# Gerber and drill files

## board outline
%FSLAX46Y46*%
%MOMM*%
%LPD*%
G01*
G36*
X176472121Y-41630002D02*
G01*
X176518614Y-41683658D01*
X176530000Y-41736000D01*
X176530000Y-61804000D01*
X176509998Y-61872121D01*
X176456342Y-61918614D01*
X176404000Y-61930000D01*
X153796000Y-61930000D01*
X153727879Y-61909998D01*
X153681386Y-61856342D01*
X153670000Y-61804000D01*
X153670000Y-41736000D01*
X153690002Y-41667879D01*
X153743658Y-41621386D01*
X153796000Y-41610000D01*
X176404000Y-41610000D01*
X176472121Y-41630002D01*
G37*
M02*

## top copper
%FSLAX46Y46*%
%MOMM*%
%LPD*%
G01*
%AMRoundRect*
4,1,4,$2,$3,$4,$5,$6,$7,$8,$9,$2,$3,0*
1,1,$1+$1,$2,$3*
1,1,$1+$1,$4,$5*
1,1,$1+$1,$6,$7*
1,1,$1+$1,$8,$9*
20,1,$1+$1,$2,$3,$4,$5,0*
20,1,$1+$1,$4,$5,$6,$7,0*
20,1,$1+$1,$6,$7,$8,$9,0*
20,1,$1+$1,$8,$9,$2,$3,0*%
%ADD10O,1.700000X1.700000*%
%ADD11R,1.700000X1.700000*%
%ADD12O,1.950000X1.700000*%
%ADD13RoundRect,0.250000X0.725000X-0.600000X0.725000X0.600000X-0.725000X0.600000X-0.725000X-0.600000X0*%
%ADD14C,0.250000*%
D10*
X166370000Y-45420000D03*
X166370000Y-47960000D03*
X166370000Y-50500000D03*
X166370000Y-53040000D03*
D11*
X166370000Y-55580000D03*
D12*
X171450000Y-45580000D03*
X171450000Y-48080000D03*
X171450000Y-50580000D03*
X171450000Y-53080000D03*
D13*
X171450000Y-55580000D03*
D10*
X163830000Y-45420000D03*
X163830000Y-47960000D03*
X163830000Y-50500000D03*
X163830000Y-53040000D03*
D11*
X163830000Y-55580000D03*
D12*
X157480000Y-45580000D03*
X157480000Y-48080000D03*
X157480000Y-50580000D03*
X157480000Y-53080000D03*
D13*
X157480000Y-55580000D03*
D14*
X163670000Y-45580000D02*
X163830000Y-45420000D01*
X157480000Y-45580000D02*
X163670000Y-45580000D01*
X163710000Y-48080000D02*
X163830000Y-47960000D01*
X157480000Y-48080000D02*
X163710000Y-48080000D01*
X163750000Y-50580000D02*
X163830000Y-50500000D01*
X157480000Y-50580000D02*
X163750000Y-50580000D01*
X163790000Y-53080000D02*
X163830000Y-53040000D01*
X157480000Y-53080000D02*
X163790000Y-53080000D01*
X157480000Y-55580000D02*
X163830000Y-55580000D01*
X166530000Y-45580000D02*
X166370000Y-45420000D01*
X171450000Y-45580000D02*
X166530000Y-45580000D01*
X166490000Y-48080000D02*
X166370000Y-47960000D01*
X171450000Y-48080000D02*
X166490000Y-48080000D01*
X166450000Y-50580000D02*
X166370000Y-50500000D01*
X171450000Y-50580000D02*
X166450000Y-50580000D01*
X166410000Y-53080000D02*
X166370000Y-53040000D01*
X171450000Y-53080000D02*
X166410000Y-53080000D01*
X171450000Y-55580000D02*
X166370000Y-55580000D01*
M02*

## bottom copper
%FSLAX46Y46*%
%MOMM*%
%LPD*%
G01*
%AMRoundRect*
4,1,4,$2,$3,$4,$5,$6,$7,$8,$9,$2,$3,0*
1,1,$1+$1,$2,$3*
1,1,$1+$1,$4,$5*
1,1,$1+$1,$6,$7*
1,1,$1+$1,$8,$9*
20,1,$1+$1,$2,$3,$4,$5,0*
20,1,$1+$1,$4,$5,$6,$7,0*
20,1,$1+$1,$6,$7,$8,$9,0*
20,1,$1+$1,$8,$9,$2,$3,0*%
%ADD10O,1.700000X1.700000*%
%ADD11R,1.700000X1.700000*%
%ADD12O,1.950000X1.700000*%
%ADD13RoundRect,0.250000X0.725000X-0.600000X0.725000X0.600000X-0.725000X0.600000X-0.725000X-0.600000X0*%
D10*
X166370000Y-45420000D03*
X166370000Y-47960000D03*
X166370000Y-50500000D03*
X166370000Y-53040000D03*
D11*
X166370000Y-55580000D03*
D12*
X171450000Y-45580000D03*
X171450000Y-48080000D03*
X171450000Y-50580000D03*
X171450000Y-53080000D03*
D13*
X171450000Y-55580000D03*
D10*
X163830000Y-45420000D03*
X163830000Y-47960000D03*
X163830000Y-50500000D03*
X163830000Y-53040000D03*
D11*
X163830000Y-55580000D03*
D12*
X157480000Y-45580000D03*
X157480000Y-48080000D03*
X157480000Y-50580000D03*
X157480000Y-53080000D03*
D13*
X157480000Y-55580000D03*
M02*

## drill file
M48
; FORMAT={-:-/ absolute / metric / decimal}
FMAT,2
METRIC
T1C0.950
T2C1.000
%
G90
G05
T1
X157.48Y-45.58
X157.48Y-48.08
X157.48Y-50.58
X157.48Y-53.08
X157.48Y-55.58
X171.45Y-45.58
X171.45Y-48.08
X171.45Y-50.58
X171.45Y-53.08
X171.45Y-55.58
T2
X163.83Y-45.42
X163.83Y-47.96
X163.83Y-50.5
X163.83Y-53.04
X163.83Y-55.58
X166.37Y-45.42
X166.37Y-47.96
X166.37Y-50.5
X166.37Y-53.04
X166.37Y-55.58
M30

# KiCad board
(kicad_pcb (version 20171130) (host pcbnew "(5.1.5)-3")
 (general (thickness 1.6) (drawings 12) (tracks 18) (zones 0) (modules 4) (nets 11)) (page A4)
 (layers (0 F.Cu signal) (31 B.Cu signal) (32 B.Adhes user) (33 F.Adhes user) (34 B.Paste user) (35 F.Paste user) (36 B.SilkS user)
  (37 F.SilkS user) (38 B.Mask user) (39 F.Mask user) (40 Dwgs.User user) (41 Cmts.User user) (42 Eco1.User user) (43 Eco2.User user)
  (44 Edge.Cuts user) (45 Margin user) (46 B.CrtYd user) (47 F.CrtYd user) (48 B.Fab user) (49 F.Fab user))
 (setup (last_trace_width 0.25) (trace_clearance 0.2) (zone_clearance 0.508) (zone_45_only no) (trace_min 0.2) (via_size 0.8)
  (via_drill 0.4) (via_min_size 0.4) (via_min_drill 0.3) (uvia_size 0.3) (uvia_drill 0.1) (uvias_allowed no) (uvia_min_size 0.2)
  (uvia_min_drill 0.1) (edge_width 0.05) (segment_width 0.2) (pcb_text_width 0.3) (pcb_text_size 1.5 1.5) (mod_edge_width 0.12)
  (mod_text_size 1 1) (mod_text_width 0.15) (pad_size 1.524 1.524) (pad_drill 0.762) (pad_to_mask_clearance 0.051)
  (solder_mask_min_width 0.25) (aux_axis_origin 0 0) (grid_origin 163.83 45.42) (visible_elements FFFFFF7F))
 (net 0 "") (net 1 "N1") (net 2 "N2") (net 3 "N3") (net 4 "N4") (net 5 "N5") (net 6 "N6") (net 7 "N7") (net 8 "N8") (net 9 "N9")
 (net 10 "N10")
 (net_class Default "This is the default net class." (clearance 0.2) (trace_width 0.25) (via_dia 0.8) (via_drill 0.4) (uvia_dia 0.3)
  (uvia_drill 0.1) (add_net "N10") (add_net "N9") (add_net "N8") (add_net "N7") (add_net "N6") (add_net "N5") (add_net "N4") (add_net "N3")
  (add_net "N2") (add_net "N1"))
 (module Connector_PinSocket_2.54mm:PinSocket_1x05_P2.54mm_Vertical (layer B.Cu) (at 166.37 55.58)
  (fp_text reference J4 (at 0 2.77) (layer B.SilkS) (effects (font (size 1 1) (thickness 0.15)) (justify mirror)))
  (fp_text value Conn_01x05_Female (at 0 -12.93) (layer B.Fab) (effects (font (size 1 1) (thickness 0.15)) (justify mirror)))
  (pad 5 thru_hole oval (at 0 -10.16) (size 1.7 1.7) (drill 1) (layers *.Cu *.Mask) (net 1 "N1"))
  (pad 4 thru_hole oval (at 0 -7.62) (size 1.7 1.7) (drill 1) (layers *.Cu *.Mask) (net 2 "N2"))
  (pad 3 thru_hole oval (at 0 -5.08) (size 1.7 1.7) (drill 1) (layers *.Cu *.Mask) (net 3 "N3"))
  (pad 2 thru_hole oval (at 0 -2.54) (size 1.7 1.7) (drill 1) (layers *.Cu *.Mask) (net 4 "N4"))
  (pad 1 thru_hole rect (at 0 0) (size 1.7 1.7) (drill 1) (layers *.Cu *.Mask) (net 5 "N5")))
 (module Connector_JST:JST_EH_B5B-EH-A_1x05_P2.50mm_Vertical (layer F.Cu) (at 171.45 55.58 90)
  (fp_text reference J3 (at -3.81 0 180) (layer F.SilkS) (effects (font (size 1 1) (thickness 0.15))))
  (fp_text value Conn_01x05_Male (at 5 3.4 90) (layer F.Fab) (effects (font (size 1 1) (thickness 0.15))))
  (pad 5 thru_hole oval (at 10 0 90) (size 1.7 1.95) (drill 0.95) (layers *.Cu *.Mask) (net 1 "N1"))
  (pad 4 thru_hole oval (at 7.5 0 90) (size 1.7 1.95) (drill 0.95) (layers *.Cu *.Mask) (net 2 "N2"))
  (pad 3 thru_hole oval (at 5 0 90) (size 1.7 1.95) (drill 0.95) (layers *.Cu *.Mask) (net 3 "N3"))
  (pad 2 thru_hole oval (at 2.5 0 90) (size 1.7 1.95) (drill 0.95) (layers *.Cu *.Mask) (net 4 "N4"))
  (pad 1 thru_hole roundrect (at 0 0 90) (size 1.7 1.95) (drill 0.95) (layers *.Cu *.Mask) (roundrect_rratio 0.147059) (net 5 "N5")))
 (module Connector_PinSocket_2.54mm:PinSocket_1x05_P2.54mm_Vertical (layer B.Cu) (at 163.83 55.58)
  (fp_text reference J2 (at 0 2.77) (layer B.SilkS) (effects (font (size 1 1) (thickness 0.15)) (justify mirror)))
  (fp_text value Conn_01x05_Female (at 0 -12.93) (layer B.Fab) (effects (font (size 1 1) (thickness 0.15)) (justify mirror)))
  (pad 5 thru_hole oval (at 0 -10.16) (size 1.7 1.7) (drill 1) (layers *.Cu *.Mask) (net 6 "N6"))
  (pad 4 thru_hole oval (at 0 -7.62) (size 1.7 1.7) (drill 1) (layers *.Cu *.Mask) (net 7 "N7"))
  (pad 3 thru_hole oval (at 0 -5.08) (size 1.7 1.7) (drill 1) (layers *.Cu *.Mask) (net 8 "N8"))
  (pad 2 thru_hole oval (at 0 -2.54) (size 1.7 1.7) (drill 1) (layers *.Cu *.Mask) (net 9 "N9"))
  (pad 1 thru_hole rect (at 0 0) (size 1.7 1.7) (drill 1) (layers *.Cu *.Mask) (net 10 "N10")))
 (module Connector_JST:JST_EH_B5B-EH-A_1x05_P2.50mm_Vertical (layer F.Cu) (at 157.48 55.58 90)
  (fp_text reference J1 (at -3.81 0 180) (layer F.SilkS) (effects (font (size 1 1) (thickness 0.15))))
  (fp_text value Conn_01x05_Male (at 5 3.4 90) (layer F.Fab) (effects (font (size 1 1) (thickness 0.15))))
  (pad 5 thru_hole oval (at 10 0 90) (size 1.7 1.95) (drill 0.95) (layers *.Cu *.Mask) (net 6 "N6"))
  (pad 4 thru_hole oval (at 7.5 0 90) (size 1.7 1.95) (drill 0.95) (layers *.Cu *.Mask) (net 7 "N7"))
  (pad 3 thru_hole oval (at 5 0 90) (size 1.7 1.95) (drill 0.95) (layers *.Cu *.Mask) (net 8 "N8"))
  (pad 2 thru_hole oval (at 2.5 0 90) (size 1.7 1.95) (drill 0.95) (layers *.Cu *.Mask) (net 9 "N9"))
  (pad 1 thru_hole roundrect (at 0 0 90) (size 1.7 1.95) (drill 0.95) (layers *.Cu *.Mask) (roundrect_rratio 0.147059) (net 10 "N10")))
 (segment (start 163.67 45.58) (end 163.83 45.42) (width 0.25) (layer F.Cu) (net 6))
 (segment (start 157.48 45.58) (end 163.67 45.58) (width 0.25) (layer F.Cu) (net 6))
 (segment (start 163.71 48.08) (end 163.83 47.96) (width 0.25) (layer F.Cu) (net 7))
 (segment (start 157.48 48.08) (end 163.71 48.08) (width 0.25) (layer F.Cu) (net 7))
 (segment (start 163.75 50.58) (end 163.83 50.5) (width 0.25) (layer F.Cu) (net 8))
 (segment (start 157.48 50.58) (end 163.75 50.58) (width 0.25) (layer F.Cu) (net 8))
 (segment (start 163.79 53.08) (end 163.83 53.04) (width 0.25) (layer F.Cu) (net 9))
 (segment (start 157.48 53.08) (end 163.79 53.08) (width 0.25) (layer F.Cu) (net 9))
 (segment (start 157.48 55.58) (end 163.83 55.58) (width 0.25) (layer F.Cu) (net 10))
 (segment (start 166.53 45.58) (end 166.37 45.42) (width 0.25) (layer F.Cu) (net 1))
 (segment (start 171.45 45.58) (end 166.53 45.58) (width 0.25) (layer F.Cu) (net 1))
 (segment (start 166.49 48.08) (end 166.37 47.96) (width 0.25) (layer F.Cu) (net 2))
 (segment (start 171.45 48.08) (end 166.49 48.08) (width 0.25) (layer F.Cu) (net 2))
 (segment (start 166.45 50.58) (end 166.37 50.5) (width 0.25) (layer F.Cu) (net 3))
 (segment (start 171.45 50.58) (end 166.45 50.58) (width 0.25) (layer F.Cu) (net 3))
 (segment (start 166.41 53.08) (end 166.37 53.04) (width 0.25) (layer F.Cu) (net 4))
 (segment (start 171.45 53.08) (end 166.41 53.08) (width 0.25) (layer F.Cu) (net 4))
 (segment (start 171.45 55.58) (end 166.37 55.58) (width 0.25) (layer F.Cu) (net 5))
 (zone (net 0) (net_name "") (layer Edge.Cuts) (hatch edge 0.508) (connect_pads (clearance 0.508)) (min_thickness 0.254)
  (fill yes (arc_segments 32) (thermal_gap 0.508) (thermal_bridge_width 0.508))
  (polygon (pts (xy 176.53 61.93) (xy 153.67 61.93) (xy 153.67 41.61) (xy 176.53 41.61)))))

